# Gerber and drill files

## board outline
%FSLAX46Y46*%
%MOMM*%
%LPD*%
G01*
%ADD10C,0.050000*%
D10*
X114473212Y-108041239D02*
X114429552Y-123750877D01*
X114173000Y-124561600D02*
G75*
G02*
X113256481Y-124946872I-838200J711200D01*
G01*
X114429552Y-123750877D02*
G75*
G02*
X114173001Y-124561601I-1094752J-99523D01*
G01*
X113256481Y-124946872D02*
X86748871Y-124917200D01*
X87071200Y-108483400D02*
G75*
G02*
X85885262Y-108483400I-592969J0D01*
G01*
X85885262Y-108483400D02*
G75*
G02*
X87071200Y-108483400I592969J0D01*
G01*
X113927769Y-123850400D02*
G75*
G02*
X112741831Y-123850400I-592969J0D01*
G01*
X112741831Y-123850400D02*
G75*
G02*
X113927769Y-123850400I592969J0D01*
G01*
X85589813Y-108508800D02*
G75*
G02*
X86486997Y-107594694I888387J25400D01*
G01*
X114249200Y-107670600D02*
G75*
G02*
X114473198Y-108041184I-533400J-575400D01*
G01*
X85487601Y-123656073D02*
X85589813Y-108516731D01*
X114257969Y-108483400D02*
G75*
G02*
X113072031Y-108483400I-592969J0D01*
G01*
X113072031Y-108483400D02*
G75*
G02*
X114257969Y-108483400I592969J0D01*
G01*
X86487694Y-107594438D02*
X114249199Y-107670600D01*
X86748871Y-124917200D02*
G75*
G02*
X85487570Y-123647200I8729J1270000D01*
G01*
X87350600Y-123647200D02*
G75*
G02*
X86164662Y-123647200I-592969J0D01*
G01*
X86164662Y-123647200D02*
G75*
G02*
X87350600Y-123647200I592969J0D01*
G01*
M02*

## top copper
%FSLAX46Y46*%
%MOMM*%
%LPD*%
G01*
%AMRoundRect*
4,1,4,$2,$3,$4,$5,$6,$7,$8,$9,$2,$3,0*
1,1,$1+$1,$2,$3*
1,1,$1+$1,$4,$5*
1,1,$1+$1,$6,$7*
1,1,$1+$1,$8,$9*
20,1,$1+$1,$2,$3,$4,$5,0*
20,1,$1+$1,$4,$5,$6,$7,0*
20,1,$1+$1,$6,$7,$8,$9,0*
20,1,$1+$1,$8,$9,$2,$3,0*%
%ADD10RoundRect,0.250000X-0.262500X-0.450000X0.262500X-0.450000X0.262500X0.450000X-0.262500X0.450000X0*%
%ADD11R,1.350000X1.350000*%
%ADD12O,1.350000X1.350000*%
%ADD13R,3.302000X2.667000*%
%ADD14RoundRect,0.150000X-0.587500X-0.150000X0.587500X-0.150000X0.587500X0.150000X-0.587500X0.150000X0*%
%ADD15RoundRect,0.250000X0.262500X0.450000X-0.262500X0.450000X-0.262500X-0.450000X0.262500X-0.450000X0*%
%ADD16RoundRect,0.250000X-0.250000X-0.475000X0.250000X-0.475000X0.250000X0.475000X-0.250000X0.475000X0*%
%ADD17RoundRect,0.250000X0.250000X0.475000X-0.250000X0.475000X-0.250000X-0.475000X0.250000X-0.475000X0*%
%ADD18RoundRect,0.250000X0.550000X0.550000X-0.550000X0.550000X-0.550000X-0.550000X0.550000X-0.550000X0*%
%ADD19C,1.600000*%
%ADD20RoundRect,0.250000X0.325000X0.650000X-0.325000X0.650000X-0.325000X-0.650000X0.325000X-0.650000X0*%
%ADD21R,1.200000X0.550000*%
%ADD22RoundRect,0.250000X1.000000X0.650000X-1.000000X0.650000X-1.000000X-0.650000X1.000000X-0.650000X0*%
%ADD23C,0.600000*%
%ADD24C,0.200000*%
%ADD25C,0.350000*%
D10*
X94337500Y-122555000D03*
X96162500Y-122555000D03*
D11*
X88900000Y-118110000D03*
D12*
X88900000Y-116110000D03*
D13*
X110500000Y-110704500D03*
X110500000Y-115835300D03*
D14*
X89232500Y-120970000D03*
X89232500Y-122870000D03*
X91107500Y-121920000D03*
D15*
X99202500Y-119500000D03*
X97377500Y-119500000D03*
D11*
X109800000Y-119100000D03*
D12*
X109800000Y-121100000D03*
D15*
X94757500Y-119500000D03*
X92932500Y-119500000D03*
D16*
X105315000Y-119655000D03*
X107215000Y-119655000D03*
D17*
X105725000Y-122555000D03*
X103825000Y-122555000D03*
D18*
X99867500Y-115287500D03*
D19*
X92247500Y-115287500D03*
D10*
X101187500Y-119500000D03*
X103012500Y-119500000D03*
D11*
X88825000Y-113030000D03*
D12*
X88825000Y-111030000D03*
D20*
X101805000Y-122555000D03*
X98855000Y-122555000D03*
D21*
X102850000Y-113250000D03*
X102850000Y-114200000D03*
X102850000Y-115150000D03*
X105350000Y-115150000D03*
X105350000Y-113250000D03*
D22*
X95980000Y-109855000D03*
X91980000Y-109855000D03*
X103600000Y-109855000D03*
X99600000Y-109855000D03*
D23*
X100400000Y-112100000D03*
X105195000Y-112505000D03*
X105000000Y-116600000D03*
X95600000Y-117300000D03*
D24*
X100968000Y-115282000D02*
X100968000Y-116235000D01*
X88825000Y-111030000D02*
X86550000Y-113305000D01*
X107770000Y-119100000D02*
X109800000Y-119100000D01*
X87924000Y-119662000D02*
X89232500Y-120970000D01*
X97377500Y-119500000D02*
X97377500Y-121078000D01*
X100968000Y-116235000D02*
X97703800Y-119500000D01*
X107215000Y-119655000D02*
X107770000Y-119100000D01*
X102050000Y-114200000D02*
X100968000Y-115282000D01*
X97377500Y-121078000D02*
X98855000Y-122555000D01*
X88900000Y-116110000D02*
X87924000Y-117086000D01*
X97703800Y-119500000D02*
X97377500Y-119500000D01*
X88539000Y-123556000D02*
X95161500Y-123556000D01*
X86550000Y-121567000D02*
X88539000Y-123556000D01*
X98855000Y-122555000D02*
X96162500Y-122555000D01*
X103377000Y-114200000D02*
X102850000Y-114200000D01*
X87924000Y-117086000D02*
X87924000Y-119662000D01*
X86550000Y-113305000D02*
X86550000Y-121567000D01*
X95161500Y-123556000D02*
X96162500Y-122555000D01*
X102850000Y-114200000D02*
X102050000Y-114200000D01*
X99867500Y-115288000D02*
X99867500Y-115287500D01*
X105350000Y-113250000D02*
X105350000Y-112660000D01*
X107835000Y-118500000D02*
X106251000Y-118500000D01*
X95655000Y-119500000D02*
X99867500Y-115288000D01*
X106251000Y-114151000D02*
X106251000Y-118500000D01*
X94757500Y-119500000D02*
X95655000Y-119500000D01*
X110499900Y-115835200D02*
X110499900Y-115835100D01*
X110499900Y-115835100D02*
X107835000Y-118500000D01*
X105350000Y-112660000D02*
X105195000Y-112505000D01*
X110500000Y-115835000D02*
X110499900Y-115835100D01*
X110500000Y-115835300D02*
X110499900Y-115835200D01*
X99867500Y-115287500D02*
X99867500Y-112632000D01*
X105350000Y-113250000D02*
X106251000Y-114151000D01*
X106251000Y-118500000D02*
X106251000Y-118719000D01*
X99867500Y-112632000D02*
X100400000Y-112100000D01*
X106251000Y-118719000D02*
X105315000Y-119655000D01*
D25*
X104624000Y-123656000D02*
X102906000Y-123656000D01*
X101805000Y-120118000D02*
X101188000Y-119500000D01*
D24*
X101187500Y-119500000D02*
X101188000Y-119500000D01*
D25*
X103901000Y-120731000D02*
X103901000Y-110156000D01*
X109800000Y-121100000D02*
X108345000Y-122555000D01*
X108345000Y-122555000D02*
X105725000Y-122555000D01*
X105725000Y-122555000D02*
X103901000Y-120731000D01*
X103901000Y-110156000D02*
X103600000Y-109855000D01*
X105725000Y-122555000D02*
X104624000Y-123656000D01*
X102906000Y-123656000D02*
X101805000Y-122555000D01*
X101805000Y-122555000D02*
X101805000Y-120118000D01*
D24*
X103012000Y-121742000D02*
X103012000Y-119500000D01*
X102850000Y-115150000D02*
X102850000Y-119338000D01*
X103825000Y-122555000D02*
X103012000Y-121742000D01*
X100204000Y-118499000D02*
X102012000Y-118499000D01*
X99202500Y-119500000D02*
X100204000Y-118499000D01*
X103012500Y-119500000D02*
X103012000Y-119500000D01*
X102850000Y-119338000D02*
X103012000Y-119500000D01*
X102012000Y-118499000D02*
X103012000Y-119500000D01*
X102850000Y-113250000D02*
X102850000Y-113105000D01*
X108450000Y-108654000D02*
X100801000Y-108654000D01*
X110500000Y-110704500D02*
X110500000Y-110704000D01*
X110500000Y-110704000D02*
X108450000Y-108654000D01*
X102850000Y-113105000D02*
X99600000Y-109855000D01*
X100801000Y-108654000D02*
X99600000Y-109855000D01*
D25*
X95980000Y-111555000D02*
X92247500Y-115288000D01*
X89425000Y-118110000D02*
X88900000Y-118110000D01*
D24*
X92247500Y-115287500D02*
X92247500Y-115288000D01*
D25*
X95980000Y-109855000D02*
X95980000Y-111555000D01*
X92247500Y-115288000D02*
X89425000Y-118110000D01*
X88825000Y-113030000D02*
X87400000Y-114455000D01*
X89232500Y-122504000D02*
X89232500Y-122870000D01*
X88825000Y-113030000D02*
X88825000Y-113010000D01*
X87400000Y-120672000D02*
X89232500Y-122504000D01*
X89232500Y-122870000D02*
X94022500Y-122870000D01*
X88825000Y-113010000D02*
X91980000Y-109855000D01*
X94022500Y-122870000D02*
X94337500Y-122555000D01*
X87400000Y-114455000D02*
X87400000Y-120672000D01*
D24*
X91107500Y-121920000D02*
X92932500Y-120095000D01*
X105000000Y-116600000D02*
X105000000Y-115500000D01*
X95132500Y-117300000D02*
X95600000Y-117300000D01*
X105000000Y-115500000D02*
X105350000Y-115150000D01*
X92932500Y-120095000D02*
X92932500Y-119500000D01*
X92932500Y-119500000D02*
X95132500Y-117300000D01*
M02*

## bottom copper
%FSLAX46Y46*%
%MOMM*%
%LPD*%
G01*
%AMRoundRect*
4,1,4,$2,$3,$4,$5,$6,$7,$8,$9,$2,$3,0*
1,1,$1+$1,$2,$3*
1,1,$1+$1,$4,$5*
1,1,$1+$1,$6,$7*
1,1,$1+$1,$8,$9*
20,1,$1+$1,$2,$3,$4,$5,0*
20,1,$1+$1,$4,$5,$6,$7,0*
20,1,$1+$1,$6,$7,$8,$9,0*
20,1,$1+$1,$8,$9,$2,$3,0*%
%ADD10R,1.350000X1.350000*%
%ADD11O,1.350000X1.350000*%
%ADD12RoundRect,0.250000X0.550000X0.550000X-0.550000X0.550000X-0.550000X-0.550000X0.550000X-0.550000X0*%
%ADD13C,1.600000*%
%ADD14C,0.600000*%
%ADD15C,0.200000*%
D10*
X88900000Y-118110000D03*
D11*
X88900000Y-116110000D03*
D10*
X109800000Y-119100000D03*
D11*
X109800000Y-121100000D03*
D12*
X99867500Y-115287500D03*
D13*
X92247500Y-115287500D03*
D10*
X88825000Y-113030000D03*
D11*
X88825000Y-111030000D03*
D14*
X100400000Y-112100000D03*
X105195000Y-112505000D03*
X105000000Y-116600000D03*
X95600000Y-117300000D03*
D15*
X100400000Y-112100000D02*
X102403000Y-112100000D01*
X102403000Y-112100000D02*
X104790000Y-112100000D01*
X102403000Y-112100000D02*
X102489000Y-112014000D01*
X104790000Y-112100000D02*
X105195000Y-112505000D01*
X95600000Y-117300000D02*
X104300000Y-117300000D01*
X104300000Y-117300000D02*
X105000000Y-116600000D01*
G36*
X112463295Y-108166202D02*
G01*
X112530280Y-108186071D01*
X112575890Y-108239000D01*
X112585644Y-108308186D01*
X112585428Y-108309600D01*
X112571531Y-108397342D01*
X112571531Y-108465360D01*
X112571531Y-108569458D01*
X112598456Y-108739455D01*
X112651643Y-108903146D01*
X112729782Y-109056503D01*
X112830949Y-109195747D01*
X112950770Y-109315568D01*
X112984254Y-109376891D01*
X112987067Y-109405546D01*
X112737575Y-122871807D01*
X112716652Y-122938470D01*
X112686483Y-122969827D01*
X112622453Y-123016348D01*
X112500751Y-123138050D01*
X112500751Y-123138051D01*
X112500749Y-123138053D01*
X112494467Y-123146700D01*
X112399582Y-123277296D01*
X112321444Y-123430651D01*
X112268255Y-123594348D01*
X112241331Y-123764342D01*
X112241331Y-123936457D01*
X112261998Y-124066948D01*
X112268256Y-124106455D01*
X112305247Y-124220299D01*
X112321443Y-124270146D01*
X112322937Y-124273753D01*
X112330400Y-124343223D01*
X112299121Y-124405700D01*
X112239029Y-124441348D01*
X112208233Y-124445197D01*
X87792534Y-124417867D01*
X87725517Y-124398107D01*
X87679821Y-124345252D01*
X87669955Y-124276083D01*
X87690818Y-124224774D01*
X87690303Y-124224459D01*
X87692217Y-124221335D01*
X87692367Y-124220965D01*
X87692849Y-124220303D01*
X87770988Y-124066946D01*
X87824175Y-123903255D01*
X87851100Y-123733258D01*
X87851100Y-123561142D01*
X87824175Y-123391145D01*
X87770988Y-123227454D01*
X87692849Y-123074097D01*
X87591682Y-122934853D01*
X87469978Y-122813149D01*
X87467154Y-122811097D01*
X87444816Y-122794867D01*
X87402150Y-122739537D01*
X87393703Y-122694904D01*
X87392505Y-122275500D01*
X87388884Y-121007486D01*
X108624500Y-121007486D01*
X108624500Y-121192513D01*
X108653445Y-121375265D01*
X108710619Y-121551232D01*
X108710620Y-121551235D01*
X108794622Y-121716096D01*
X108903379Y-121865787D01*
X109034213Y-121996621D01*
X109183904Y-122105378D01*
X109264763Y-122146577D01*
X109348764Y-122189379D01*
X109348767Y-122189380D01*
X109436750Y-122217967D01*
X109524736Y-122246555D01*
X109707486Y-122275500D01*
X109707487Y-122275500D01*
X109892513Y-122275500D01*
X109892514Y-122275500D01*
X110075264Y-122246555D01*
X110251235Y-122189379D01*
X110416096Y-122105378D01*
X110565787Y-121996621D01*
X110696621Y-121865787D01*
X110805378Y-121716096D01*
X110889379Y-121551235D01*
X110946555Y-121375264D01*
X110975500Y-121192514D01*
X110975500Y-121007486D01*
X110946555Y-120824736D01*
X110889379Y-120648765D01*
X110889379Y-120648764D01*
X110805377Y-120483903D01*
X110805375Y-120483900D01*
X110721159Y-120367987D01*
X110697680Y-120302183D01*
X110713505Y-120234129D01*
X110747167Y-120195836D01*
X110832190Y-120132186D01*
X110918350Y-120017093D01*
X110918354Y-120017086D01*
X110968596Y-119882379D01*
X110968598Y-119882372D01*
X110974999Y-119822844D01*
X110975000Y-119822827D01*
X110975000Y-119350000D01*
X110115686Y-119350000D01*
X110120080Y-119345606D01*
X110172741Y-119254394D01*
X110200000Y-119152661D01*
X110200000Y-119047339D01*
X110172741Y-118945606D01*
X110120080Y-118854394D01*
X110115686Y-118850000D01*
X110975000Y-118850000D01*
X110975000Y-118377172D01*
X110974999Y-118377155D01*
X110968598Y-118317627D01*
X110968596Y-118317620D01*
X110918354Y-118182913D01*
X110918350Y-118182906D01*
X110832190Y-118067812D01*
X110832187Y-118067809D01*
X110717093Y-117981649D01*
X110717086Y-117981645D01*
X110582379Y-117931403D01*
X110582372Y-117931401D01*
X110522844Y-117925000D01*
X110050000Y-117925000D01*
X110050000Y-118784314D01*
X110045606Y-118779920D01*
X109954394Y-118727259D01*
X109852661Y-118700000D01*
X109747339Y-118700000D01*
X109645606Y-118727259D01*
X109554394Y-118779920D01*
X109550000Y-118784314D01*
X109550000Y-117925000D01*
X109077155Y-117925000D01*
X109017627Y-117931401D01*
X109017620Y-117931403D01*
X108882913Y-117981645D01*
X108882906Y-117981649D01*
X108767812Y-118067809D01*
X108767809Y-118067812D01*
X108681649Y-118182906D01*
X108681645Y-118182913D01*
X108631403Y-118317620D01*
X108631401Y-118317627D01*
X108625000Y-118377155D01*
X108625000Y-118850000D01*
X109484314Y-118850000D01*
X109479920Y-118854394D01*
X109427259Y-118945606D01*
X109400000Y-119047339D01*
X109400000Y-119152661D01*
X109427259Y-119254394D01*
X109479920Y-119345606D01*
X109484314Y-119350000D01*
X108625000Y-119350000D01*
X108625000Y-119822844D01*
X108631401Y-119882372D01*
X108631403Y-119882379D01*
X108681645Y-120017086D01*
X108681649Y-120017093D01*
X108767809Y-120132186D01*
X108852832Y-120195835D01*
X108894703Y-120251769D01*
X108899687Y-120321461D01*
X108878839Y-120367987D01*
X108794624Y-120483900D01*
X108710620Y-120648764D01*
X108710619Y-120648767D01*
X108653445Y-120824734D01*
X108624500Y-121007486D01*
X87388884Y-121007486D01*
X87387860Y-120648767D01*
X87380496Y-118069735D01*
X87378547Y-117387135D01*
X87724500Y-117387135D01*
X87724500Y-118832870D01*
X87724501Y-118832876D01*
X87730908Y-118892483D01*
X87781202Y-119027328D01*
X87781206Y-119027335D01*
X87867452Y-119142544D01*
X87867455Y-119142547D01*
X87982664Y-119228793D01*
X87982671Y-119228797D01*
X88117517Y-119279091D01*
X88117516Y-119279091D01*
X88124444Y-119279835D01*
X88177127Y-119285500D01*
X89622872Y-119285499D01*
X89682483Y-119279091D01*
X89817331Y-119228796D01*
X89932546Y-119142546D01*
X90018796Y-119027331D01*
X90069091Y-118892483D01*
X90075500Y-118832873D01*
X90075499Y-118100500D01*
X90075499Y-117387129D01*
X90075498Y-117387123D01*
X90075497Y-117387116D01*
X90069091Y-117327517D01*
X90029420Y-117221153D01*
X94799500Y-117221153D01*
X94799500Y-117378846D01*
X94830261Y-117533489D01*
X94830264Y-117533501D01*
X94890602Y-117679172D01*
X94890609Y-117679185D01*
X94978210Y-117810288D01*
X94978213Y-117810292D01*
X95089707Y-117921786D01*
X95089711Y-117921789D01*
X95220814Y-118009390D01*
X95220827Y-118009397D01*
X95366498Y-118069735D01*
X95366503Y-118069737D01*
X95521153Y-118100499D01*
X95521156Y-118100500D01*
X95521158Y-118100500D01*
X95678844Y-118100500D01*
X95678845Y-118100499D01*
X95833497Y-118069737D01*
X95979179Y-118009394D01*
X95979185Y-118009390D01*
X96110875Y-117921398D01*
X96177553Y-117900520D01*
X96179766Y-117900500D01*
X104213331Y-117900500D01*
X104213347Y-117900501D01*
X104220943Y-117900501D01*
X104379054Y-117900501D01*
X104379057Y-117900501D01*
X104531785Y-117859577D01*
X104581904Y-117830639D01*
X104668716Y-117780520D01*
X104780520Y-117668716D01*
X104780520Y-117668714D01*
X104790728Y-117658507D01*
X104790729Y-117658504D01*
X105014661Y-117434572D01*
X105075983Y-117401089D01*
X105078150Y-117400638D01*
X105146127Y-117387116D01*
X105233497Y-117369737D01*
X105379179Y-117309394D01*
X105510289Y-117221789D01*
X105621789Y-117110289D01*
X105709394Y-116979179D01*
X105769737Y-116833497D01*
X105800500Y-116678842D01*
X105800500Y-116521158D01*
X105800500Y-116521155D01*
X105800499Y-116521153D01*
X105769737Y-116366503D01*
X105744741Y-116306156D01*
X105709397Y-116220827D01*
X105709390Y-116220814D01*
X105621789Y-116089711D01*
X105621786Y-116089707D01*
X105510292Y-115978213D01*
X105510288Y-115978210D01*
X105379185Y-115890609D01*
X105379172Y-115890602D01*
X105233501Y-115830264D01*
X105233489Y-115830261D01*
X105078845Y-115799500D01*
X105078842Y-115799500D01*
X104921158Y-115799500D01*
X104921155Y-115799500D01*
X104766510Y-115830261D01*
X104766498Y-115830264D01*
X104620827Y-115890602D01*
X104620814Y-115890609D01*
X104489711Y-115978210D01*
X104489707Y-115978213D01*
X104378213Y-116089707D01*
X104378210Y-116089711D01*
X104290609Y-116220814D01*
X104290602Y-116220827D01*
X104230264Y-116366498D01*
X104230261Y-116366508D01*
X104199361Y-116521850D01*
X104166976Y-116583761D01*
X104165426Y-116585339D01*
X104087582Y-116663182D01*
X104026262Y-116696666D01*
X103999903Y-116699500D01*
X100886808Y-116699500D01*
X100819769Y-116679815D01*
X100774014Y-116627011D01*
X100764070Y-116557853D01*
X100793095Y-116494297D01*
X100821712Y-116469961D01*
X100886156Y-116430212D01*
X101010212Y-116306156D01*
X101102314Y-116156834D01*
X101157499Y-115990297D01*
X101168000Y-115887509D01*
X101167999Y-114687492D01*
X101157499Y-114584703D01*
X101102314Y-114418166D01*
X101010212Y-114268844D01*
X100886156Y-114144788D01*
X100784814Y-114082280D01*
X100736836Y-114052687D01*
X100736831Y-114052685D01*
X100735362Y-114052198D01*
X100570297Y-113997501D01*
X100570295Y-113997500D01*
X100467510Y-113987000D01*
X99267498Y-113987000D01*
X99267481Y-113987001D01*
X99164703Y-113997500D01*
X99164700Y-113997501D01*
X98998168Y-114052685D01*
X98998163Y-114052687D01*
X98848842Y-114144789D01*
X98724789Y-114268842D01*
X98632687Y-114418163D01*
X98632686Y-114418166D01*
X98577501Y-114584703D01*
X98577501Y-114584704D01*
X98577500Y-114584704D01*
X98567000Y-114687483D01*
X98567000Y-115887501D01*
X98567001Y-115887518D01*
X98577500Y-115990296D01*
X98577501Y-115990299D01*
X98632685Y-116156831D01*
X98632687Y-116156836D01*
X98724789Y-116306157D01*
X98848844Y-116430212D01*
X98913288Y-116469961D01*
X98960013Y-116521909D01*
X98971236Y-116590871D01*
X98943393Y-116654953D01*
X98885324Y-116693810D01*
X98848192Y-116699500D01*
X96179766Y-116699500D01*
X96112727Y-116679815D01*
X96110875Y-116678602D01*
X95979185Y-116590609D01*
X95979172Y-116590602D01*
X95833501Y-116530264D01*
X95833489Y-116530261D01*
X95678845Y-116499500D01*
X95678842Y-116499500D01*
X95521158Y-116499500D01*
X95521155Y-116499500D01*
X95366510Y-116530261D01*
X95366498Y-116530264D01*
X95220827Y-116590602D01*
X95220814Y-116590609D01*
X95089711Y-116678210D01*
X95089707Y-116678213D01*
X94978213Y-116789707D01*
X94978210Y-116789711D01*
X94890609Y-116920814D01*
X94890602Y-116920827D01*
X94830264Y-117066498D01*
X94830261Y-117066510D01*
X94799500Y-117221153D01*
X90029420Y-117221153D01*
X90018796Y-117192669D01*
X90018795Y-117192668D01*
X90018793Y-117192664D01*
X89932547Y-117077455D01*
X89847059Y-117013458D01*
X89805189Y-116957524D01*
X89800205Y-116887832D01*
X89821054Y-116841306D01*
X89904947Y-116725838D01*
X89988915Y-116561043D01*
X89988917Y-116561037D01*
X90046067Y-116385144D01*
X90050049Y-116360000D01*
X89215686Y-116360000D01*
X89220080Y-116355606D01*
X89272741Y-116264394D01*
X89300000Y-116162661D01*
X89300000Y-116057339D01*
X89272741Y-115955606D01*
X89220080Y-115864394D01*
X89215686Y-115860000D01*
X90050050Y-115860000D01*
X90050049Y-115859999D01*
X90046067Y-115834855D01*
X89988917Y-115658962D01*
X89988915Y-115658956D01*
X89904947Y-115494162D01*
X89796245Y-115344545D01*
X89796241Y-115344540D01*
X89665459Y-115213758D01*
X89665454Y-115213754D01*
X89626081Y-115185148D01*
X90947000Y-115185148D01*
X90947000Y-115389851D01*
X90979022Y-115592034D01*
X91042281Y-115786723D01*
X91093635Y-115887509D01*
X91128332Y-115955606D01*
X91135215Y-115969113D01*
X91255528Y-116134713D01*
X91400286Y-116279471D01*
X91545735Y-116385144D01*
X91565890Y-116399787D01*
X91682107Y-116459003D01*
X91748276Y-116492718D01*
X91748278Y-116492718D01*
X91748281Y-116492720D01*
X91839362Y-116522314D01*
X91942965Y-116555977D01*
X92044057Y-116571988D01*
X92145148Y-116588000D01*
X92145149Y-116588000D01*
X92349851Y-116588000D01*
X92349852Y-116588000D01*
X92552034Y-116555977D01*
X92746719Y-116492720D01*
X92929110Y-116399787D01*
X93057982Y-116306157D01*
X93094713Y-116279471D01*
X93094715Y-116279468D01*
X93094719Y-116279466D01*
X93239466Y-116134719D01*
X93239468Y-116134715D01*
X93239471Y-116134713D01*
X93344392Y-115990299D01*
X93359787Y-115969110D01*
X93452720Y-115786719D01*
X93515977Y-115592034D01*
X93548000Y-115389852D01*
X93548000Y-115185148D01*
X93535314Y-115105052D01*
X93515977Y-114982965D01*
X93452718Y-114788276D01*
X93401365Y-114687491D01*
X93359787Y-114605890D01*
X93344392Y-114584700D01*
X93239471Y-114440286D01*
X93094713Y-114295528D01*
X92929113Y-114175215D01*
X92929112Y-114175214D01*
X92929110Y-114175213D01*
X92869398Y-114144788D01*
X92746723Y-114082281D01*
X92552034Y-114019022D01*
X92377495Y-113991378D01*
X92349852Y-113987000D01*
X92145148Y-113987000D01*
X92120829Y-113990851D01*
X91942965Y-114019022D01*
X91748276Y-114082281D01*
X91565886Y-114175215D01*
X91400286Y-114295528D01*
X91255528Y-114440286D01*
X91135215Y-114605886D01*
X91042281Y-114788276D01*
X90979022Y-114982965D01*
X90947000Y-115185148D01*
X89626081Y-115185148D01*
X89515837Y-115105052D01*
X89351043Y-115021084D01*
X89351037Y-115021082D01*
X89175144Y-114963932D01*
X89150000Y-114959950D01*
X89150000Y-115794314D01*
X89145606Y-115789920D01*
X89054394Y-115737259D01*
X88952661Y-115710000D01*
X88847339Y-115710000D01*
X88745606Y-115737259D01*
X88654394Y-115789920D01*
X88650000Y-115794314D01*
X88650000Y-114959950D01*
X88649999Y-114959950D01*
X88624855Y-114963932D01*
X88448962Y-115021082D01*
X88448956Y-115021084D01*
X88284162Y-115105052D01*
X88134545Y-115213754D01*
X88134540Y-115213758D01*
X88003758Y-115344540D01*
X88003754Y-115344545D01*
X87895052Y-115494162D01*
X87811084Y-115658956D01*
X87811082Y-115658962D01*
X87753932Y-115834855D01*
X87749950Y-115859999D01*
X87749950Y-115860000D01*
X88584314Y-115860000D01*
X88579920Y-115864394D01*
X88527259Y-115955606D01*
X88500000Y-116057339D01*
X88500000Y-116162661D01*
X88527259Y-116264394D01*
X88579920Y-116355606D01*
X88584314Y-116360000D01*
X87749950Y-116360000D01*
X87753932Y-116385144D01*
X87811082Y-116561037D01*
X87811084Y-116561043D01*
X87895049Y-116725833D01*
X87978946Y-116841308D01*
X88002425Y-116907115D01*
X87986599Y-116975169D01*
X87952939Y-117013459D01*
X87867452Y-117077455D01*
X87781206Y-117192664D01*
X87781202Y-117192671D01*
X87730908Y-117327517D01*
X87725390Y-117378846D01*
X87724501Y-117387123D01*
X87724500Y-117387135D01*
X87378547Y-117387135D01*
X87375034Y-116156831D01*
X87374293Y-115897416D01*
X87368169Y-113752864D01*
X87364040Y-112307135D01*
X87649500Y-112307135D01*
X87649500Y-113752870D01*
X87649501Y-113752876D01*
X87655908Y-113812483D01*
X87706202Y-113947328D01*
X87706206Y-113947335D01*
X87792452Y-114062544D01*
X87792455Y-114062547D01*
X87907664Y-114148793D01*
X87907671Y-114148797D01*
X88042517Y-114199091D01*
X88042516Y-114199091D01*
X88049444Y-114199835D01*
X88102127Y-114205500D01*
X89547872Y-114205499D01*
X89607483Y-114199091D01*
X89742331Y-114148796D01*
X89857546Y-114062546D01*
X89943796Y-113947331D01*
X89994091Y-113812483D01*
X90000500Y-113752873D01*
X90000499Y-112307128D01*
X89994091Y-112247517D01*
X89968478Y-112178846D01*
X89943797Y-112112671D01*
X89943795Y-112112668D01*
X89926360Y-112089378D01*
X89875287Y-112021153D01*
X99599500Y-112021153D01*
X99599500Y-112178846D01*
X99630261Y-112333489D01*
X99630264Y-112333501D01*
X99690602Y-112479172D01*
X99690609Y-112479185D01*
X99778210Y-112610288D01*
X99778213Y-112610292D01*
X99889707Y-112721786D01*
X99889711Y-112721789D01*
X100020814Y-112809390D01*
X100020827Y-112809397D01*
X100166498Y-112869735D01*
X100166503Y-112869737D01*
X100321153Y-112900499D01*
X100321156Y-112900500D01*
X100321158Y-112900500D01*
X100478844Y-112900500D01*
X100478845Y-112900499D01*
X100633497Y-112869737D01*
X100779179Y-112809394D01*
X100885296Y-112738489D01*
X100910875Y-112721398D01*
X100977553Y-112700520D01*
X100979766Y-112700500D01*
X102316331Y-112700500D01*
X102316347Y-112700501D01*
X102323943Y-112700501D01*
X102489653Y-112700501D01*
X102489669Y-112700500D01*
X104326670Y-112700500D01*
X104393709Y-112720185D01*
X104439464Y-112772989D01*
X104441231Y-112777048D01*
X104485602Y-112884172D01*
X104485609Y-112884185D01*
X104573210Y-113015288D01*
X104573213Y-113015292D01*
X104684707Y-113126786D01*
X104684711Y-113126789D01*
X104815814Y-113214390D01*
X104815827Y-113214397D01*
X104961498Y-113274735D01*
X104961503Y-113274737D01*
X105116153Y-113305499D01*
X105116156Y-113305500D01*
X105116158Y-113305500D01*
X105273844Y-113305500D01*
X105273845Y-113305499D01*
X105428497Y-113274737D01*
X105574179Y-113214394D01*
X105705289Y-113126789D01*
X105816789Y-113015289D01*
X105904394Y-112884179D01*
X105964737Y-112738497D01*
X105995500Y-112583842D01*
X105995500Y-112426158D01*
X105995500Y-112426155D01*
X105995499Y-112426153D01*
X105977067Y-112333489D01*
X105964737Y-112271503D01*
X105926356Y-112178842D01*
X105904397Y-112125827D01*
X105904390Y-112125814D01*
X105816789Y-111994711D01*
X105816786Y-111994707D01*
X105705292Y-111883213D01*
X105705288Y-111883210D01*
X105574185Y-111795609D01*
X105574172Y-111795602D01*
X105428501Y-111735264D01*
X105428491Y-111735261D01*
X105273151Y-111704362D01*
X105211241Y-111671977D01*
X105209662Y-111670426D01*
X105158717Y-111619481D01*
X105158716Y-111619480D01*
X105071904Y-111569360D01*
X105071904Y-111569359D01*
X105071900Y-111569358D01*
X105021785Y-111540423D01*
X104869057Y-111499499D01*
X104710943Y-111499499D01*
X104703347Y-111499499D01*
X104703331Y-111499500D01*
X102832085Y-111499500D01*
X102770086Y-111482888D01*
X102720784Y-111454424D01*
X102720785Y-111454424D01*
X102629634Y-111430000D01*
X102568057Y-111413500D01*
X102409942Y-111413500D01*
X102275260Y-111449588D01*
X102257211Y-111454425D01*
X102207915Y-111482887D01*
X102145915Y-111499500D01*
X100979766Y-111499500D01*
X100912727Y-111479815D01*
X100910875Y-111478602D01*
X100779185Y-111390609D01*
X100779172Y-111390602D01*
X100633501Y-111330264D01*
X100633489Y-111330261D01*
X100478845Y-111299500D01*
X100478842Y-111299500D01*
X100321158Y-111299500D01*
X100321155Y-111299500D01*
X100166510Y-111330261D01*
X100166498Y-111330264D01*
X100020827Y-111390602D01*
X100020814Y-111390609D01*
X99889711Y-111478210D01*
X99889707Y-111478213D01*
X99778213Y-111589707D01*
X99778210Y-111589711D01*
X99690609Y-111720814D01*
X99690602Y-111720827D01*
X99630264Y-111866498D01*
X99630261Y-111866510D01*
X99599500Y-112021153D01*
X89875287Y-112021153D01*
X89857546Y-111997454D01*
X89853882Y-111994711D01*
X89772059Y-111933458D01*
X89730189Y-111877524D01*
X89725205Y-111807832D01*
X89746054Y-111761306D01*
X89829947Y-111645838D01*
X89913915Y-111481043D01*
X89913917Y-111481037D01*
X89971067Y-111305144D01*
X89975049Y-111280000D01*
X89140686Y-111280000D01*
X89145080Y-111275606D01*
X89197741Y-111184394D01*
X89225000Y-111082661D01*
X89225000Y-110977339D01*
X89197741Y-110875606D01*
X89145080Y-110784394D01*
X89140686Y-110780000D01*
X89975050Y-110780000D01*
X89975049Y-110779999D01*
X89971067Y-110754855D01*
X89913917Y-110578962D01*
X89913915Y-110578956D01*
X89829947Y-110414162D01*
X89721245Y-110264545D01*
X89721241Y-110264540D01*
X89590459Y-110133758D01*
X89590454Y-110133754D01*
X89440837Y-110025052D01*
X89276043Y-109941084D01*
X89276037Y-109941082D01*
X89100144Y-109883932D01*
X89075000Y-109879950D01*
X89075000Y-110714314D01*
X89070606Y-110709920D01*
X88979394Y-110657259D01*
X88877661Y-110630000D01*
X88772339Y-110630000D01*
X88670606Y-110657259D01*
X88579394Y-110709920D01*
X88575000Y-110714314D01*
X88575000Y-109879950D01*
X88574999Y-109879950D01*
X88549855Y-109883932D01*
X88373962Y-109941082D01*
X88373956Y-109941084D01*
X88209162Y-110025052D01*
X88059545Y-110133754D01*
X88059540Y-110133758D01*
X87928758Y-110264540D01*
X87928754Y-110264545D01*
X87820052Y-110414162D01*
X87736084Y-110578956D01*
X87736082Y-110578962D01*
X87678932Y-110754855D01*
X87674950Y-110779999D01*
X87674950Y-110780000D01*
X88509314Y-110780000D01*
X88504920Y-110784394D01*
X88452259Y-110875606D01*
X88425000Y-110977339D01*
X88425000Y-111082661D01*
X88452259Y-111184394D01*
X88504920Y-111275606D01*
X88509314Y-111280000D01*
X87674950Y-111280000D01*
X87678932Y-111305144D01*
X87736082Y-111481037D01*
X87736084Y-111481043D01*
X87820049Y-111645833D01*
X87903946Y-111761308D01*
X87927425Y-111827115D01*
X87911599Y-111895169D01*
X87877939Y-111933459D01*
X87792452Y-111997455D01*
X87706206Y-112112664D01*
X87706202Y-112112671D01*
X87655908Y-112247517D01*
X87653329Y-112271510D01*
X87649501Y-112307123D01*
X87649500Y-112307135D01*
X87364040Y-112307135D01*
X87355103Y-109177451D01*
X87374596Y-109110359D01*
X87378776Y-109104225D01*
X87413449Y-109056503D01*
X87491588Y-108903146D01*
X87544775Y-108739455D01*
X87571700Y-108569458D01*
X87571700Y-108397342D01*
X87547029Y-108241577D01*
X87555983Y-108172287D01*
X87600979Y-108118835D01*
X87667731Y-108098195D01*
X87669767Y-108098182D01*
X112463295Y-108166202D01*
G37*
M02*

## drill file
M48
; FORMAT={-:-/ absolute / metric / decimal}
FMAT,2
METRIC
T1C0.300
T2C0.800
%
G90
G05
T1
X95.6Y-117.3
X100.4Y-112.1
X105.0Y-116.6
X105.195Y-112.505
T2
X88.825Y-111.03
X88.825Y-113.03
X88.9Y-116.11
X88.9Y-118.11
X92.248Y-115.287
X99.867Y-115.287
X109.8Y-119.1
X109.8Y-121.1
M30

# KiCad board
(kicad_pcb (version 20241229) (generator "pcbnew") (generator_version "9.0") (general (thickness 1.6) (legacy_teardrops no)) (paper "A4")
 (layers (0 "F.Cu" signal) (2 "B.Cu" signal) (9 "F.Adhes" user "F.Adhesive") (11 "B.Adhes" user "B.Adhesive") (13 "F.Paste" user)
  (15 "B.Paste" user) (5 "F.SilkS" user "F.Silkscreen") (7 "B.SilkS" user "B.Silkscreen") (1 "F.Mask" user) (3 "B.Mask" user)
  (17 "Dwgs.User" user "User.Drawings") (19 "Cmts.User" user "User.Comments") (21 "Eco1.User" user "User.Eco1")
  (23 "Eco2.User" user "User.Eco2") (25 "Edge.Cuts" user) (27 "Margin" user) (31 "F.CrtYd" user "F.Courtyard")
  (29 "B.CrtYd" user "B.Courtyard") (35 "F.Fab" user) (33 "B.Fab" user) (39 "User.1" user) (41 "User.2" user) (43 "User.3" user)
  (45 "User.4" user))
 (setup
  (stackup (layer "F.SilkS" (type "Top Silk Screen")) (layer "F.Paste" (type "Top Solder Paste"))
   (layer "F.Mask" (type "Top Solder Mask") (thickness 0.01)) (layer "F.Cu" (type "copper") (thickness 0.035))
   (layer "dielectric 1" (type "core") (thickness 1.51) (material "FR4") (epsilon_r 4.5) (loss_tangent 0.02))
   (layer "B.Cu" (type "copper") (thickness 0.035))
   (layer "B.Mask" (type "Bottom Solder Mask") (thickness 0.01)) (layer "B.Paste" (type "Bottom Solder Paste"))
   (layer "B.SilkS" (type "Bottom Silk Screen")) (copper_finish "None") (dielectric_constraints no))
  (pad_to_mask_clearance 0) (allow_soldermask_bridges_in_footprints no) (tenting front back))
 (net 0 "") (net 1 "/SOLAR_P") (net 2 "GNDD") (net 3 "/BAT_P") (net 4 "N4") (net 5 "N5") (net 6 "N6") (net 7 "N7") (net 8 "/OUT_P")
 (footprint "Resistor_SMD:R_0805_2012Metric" (layer "F.Cu") (at 95.25 122.555)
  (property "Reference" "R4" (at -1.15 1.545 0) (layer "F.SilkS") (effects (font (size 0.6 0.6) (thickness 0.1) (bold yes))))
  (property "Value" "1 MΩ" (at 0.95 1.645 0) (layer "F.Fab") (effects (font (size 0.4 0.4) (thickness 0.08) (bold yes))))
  (pad "1" smd roundrect (at -0.9125 0) (size 1.025 1.4) (layers "F.Cu" "F.Mask" "F.Paste") (roundrect_rratio 0.243902) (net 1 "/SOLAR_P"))
  (pad "2" smd roundrect (at 0.9125 0) (size 1.025 1.4) (layers "F.Cu" "F.Mask" "F.Paste") (roundrect_rratio 0.243902) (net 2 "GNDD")))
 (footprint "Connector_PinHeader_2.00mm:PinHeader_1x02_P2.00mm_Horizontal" (layer "F.Cu") (at 88.9 118.11 180)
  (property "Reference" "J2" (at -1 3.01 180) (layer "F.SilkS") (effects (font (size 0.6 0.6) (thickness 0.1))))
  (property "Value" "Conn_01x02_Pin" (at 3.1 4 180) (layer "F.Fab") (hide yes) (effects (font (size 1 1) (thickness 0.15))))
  (pad "1" thru_hole rect (at 0 0 180) (size 1.35 1.35) (drill 0.8) (layers "*.Cu" "*.Mask") (remove_unused_layers no) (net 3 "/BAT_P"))
  (pad "2" thru_hole oval (at 0 2 180) (size 1.35 1.35) (drill 0.8) (layers "*.Cu" "*.Mask") (remove_unused_layers no) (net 2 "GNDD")))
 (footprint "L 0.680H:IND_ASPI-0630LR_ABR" (layer "F.Cu") (at 110.5 113.2699 -90)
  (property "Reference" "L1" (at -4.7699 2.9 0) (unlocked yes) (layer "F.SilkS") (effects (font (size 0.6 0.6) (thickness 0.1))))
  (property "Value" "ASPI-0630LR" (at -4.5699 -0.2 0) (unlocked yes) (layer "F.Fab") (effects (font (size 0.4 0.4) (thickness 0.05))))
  (pad "1" smd rect (at -2.5654 0) (size 3.302 2.667) (layers "F.Cu" "F.Mask" "F.Paste") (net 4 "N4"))
  (pad "2" smd rect (at 2.5654 0) (size 3.302 2.667) (layers "F.Cu" "F.Mask" "F.Paste") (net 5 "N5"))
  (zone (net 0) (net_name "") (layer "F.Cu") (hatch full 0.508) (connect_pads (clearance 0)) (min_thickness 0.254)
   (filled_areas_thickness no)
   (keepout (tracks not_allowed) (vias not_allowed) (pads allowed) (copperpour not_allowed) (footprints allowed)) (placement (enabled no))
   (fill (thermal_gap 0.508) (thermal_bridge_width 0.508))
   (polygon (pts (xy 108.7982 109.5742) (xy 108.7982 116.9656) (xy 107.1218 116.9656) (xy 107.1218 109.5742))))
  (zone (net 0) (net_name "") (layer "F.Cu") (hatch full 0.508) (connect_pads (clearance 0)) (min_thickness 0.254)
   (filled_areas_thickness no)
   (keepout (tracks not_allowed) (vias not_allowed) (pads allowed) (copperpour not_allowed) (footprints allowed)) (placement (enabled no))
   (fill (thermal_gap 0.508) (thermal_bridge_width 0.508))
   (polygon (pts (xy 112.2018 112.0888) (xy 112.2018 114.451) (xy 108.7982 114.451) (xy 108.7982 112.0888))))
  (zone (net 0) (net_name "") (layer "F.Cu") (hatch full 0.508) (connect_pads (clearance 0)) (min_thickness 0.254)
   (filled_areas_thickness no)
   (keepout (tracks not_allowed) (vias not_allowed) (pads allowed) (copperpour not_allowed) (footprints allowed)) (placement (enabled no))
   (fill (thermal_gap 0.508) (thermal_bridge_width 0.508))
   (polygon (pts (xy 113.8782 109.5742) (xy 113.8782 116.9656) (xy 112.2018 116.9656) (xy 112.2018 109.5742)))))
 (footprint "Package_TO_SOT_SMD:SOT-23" (layer "F.Cu") (at 90.17 121.92)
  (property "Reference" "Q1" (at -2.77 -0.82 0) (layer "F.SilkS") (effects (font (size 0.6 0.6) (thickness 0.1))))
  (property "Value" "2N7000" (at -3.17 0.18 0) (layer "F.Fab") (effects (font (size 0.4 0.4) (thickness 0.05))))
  (pad "1" smd roundrect (at -0.9375 -0.95) (size 1.475 0.6) (layers "F.Cu" "F.Mask" "F.Paste") (roundrect_rratio 0.25) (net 2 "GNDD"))
  (pad "2" smd roundrect (at -0.9375 0.95) (size 1.475 0.6) (layers "F.Cu" "F.Mask" "F.Paste") (roundrect_rratio 0.25) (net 1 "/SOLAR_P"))
  (pad "3" smd roundrect (at 0.9375 0) (size 1.475 0.6) (layers "F.Cu" "F.Mask" "F.Paste") (roundrect_rratio 0.25) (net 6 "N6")))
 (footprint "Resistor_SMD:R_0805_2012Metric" (layer "F.Cu") (at 98.29 119.5 180)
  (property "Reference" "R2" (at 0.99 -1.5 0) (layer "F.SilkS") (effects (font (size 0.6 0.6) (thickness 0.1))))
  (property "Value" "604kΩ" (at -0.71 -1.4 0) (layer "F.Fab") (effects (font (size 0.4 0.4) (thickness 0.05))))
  (pad "1" smd roundrect (at -0.9125 0 180) (size 1.025 1.4) (layers "F.Cu" "F.Mask" "F.Paste") (roundrect_rratio 0.243902) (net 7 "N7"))
  (pad "2" smd roundrect (at 0.9125 0 180) (size 1.025 1.4) (layers "F.Cu" "F.Mask" "F.Paste") (roundrect_rratio 0.243902) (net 2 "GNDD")))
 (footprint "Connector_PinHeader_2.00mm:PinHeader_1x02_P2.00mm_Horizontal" (layer "F.Cu") (at 109.8 119.1)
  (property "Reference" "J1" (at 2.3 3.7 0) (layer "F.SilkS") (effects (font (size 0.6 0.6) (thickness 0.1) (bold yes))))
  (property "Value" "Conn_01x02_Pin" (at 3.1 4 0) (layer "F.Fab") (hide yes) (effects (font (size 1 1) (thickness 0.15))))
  (pad "1" thru_hole rect (at 0 0) (size 1.35 1.35) (drill 0.8) (layers "*.Cu" "*.Mask") (remove_unused_layers no) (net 2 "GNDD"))
  (pad "2" thru_hole oval (at 0 2) (size 1.35 1.35) (drill 0.8) (layers "*.Cu" "*.Mask") (remove_unused_layers no) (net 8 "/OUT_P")))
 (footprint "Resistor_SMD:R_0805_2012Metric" (layer "F.Cu") (at 93.845 119.5 180)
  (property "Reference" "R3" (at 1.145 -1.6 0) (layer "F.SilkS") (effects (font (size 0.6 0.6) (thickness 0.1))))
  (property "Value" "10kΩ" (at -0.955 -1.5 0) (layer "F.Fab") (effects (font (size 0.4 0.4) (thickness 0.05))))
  (pad "1" smd roundrect (at -0.9125 0 180) (size 1.025 1.4) (layers "F.Cu" "F.Mask" "F.Paste") (roundrect_rratio 0.243902) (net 5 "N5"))
  (pad "2" smd roundrect (at 0.9125 0 180) (size 1.025 1.4) (layers "F.Cu" "F.Mask" "F.Paste") (roundrect_rratio 0.243902) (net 6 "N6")))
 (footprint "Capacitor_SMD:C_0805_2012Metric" (layer "F.Cu") (at 106.265 119.655)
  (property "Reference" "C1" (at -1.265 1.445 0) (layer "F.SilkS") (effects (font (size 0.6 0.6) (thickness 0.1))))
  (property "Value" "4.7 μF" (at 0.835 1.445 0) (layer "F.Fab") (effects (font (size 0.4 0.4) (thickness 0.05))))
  (pad "1" smd roundrect (at -0.95 0) (size 1 1.45) (layers "F.Cu" "F.Mask" "F.Paste") (roundrect_rratio 0.25) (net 5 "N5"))
  (pad "2" smd roundrect (at 0.95 0) (size 1 1.45) (layers "F.Cu" "F.Mask" "F.Paste") (roundrect_rratio 0.25) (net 2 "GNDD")))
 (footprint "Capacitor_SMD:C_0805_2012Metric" (layer "F.Cu") (at 104.775 122.555 180)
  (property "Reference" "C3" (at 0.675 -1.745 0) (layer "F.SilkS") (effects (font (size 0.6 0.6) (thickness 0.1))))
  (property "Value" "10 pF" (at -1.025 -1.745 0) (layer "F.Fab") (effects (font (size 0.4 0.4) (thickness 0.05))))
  (pad "1" smd roundrect (at -0.95 0 180) (size 1 1.45) (layers "F.Cu" "F.Mask" "F.Paste") (roundrect_rratio 0.25) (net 8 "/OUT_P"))
  (pad "2" smd roundrect (at 0.95 0 180) (size 1 1.45) (layers "F.Cu" "F.Mask" "F.Paste") (roundrect_rratio 0.25) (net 7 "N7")))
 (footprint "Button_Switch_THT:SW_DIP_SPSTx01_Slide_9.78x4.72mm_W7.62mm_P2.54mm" (layer "F.Cu") (at 99.8675 115.2875 180)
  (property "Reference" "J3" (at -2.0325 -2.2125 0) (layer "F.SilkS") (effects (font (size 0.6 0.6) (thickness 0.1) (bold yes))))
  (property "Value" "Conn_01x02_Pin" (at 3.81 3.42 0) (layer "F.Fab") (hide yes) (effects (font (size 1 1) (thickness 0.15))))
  (pad "1" thru_hole roundrect (at 0 0 180) (size 1.6 1.6) (drill 0.8) (layers "*.Cu" "*.Mask") (remove_unused_layers no)
   (roundrect_rratio 0.15625) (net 5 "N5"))
  (pad "2" thru_hole circle (at 7.62 0 180) (size 1.6 1.6) (drill 0.8) (layers "*.Cu" "*.Mask") (remove_unused_layers no) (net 3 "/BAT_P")))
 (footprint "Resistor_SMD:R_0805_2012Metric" (layer "F.Cu") (at 102.1 119.5)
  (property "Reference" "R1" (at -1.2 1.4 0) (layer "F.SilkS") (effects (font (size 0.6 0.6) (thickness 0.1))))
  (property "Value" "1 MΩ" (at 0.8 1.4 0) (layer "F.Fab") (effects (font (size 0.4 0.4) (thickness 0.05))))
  (pad "1" smd roundrect (at -0.9125 0) (size 1.025 1.4) (layers "F.Cu" "F.Mask" "F.Paste") (roundrect_rratio 0.243902) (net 8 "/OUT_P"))
  (pad "2" smd roundrect (at 0.9125 0) (size 1.025 1.4) (layers "F.Cu" "F.Mask" "F.Paste") (roundrect_rratio 0.243902) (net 7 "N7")))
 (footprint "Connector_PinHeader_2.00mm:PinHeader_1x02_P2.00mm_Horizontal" (layer "F.Cu") (at 88.825 113.03 180)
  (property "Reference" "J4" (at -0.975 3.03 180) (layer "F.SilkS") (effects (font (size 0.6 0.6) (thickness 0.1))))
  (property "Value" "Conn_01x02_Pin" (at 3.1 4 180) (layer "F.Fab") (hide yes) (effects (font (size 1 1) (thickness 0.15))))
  (pad "1" thru_hole rect (at 0 0 180) (size 1.35 1.35) (drill 0.8) (layers "*.Cu" "*.Mask") (remove_unused_layers no) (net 1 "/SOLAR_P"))
  (pad "2" thru_hole oval (at 0 2 180) (size 1.35 1.35) (drill 0.8) (layers "*.Cu" "*.Mask") (remove_unused_layers no) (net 2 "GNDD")))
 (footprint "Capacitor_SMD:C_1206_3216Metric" (layer "F.Cu") (at 100.33 122.555 180)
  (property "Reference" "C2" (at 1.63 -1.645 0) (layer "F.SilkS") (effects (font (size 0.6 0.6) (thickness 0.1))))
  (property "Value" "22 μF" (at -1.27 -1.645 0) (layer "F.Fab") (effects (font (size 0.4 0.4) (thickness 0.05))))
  (pad "1" smd roundrect (at -1.475 0 180) (size 1.15 1.8) (layers "F.Cu" "F.Mask" "F.Paste") (roundrect_rratio 0.217391) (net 8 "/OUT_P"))
  (pad "2" smd roundrect (at 1.475 0 180) (size 1.15 1.8) (layers "F.Cu" "F.Mask" "F.Paste") (roundrect_rratio 0.217391) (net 2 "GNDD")))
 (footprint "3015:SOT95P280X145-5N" (layer "F.Cu") (at 104.1 114.2)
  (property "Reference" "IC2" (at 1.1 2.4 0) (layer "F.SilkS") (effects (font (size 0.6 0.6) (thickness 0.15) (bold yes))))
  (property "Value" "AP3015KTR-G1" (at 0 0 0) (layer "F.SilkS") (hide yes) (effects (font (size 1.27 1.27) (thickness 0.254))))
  (pad "1" smd rect (at -1.25 -0.95 90) (size 0.55 1.2) (layers "F.Cu" "F.Mask" "F.Paste") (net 4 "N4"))
  (pad "2" smd rect (at -1.25 0 90) (size 0.55 1.2) (layers "F.Cu" "F.Mask" "F.Paste") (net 2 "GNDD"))
  (pad "3" smd rect (at -1.25 0.95 90) (size 0.55 1.2) (layers "F.Cu" "F.Mask" "F.Paste") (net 7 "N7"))
  (pad "4" smd rect (at 1.25 0.95 90) (size 0.55 1.2) (layers "F.Cu" "F.Mask" "F.Paste") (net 6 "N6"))
  (pad "5" smd rect (at 1.25 -0.95 90) (size 0.55 1.2) (layers "F.Cu" "F.Mask" "F.Paste") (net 5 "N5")))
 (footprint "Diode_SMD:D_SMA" (layer "F.Cu") (at 93.98 109.855 180)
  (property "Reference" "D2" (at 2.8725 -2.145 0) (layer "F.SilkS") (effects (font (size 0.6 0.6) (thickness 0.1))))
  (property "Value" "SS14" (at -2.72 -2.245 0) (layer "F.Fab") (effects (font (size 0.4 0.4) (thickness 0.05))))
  (pad "1" smd roundrect (at -2 0 180) (size 2.5 1.8) (layers "F.Cu" "F.Mask" "F.Paste") (roundrect_rratio 0.1388888889) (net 3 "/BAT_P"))
  (pad "2" smd roundrect (at 2 0 180) (size 2.5 1.8) (layers "F.Cu" "F.Mask" "F.Paste") (roundrect_rratio 0.1388888889) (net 1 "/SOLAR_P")))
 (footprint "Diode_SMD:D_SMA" (layer "F.Cu") (at 101.6 109.855 180)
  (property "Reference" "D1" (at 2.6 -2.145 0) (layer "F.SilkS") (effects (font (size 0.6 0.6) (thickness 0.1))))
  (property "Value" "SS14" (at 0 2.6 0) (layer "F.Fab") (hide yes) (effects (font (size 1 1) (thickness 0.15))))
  (pad "1" smd roundrect (at -2 0 180) (size 2.5 1.8) (layers "F.Cu" "F.Mask" "F.Paste") (roundrect_rratio 0.1388888889) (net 8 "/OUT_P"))
  (pad "2" smd roundrect (at 2 0 180) (size 2.5 1.8) (layers "F.Cu" "F.Mask" "F.Paste") (roundrect_rratio 0.1388888889) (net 4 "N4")))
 (gr_line (start 114.473212 108.041239) (end 114.429552 123.750877) (stroke (width 0.05) (type default)) (layer "Edge.Cuts"))
 (gr_arc (start 114.173 124.5616) (mid 113.760785 124.863771) (end 113.256481 124.946872) (stroke (width 0.05) (type default))
  (layer "Edge.Cuts"))
 (gr_arc (start 114.429552 123.750877) (mid 114.382843 124.18205) (end 114.173 124.5616) (stroke (width 0.05) (type default))
  (layer "Edge.Cuts"))
 (gr_line (start 113.256481 124.946872) (end 86.748871 124.9172) (stroke (width 0.05) (type default)) (layer "Edge.Cuts"))
 (gr_circle (center 86.478231 108.4834) (end 86.884631 108.9152) (stroke (width 0.05) (type default)) (fill no) (layer "Edge.Cuts"))
 (gr_circle (center 113.3348 123.8504) (end 113.7412 124.2822) (stroke (width 0.05) (type default)) (fill no) (layer "Edge.Cuts"))
 (gr_arc (start 85.589813 108.5088) (mid 85.843913 107.860847) (end 86.486997 107.594662) (stroke (width 0.05) (type default))
  (layer "Edge.Cuts"))
 (gr_arc (start 114.2492 107.6706) (mid 114.387277 107.84013) (end 114.473212 108.04118) (stroke (width 0.05) (type default))
  (layer "Edge.Cuts"))
 (gr_line (start 85.487601 123.656073) (end 85.589813 108.516731) (stroke (width 0.05) (type default)) (layer "Edge.Cuts"))
 (gr_circle (center 113.665 108.4834) (end 114.0714 108.9152) (stroke (width 0.05) (type default)) (fill no) (layer "Edge.Cuts"))
 (gr_line (start 86.487694 107.594438) (end 114.249199 107.6706) (stroke (width 0.05) (type default)) (layer "Edge.Cuts"))
 (gr_arc (start 86.748871 124.9172) (mid 85.856492 124.542144) (end 85.487601 123.6472) (stroke (width 0.05) (type default))
  (layer "Edge.Cuts"))
 (gr_circle (center 86.757631 123.6472) (end 87.164031 124.079) (stroke (width 0.05) (type default)) (fill no) (layer "Edge.Cuts"))
 (segment (start 100.968 115.282) (end 100.968 116.235) (width 0.2) (layer "F.Cu") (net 2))
 (segment (start 88.825 111.03) (end 86.55 113.305) (width 0.2) (layer "F.Cu") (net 2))
 (segment (start 107.77 119.1) (end 109.8 119.1) (width 0.2) (layer "F.Cu") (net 2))
 (segment (start 87.924 119.662) (end 89.2325 120.97) (width 0.2) (layer "F.Cu") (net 2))
 (segment (start 97.3775 119.5) (end 97.3775 121.078) (width 0.2) (layer "F.Cu") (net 2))
 (segment (start 100.968 116.235) (end 97.7038 119.5) (width 0.2) (layer "F.Cu") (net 2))
 (segment (start 107.215 119.655) (end 107.77 119.1) (width 0.2) (layer "F.Cu") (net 2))
 (segment (start 102.05 114.2) (end 100.968 115.282) (width 0.2) (layer "F.Cu") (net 2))
 (segment (start 97.3775 121.078) (end 98.855 122.555) (width 0.2) (layer "F.Cu") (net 2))
 (segment (start 88.9 116.11) (end 87.924 117.086) (width 0.2) (layer "F.Cu") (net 2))
 (segment (start 97.7038 119.5) (end 97.3775 119.5) (width 0.2) (layer "F.Cu") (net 2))
 (segment (start 88.539 123.556) (end 95.1615 123.556) (width 0.2) (layer "F.Cu") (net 2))
 (segment (start 86.55 121.567) (end 88.539 123.556) (width 0.2) (layer "F.Cu") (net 2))
 (segment (start 98.855 122.555) (end 96.1625 122.555) (width 0.2) (layer "F.Cu") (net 2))
 (segment (start 103.377 114.2) (end 102.85 114.2) (width 0.2) (layer "F.Cu") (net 2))
 (segment (start 87.924 117.086) (end 87.924 119.662) (width 0.2) (layer "F.Cu") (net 2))
 (segment (start 86.55 113.305) (end 86.55 121.567) (width 0.2) (layer "F.Cu") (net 2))
 (segment (start 95.1615 123.556) (end 96.1625 122.555) (width 0.2) (layer "F.Cu") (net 2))
 (segment (start 102.85 114.2) (end 102.05 114.2) (width 0.2) (layer "F.Cu") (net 2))
 (segment (start 99.8675 115.288) (end 99.8675 115.2875) (width 0.2) (layer "F.Cu") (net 5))
 (segment (start 105.35 113.25) (end 105.35 112.66) (width 0.2) (layer "F.Cu") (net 5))
 (segment (start 107.835 118.5) (end 106.251 118.5) (width 0.2) (layer "F.Cu") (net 5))
 (segment (start 95.655 119.5) (end 99.8675 115.288) (width 0.2) (layer "F.Cu") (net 5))
 (segment (start 106.251 114.151) (end 106.251 118.5) (width 0.2) (layer "F.Cu") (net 5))
 (segment (start 94.7575 119.5) (end 95.655 119.5) (width 0.2) (layer "F.Cu") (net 5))
 (segment (start 110.4999 115.8352) (end 110.4999 115.8351) (width 0.2) (layer "F.Cu") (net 5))
 (segment (start 110.4999 115.8351) (end 107.835 118.5) (width 0.2) (layer "F.Cu") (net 5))
 (segment (start 105.35 112.66) (end 105.195 112.505) (width 0.2) (layer "F.Cu") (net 5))
 (segment (start 110.5 115.835) (end 110.4999 115.8351) (width 0.2) (layer "F.Cu") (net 5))
 (segment (start 110.5 115.8353) (end 110.4999 115.8352) (width 0.2) (layer "F.Cu") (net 5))
 (segment (start 99.8675 115.2875) (end 99.8675 112.632) (width 0.2) (layer "F.Cu") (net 5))
 (segment (start 105.35 113.25) (end 106.251 114.151) (width 0.2) (layer "F.Cu") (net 5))
 (segment (start 106.251 118.5) (end 106.251 118.719) (width 0.2) (layer "F.Cu") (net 5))
 (segment (start 99.8675 112.632) (end 100.4 112.1) (width 0.2) (layer "F.Cu") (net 5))
 (segment (start 106.251 118.719) (end 105.315 119.655) (width 0.2) (layer "F.Cu") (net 5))
 (via (at 100.4 112.1) (size 0.6) (drill 0.3) (layers "F.Cu" "B.Cu") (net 5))
 (via (at 105.195 112.505) (size 0.6) (drill 0.3) (layers "F.Cu" "B.Cu") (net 5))
 (segment (start 100.4 112.1) (end 102.403 112.1) (width 0.2) (layer "B.Cu") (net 5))
 (segment (start 102.403 112.1) (end 104.79 112.1) (width 0.2) (layer "B.Cu") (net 5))
 (segment (start 102.403 112.1) (end 102.489 112.014) (width 0.2) (layer "B.Cu") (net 5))
 (segment (start 104.79 112.1) (end 105.195 112.505) (width 0.2) (layer "B.Cu") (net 5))
 (segment (start 104.624 123.656) (end 102.906 123.656) (width 0.35) (layer "F.Cu") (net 8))
 (segment (start 101.805 120.118) (end 101.188 119.5) (width 0.35) (layer "F.Cu") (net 8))
 (segment (start 101.1875 119.5) (end 101.188 119.5) (width 0.2) (layer "F.Cu") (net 8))
 (segment (start 103.901 120.731) (end 103.901 110.156) (width 0.35) (layer "F.Cu") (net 8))
 (segment (start 109.8 121.1) (end 108.345 122.555) (width 0.35) (layer "F.Cu") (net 8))
 (segment (start 108.345 122.555) (end 105.725 122.555) (width 0.35) (layer "F.Cu") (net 8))
 (segment (start 105.725 122.555) (end 103.901 120.731) (width 0.35) (layer "F.Cu") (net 8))
 (segment (start 103.901 110.156) (end 103.6 109.855) (width 0.35) (layer "F.Cu") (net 8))
 (segment (start 105.725 122.555) (end 104.624 123.656) (width 0.35) (layer "F.Cu") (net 8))
 (segment (start 102.906 123.656) (end 101.805 122.555) (width 0.35) (layer "F.Cu") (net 8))
 (segment (start 101.805 122.555) (end 101.805 120.118) (width 0.35) (layer "F.Cu") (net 8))
 (segment (start 103.012 121.742) (end 103.012 119.5) (width 0.2) (layer "F.Cu") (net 7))
 (segment (start 102.85 115.15) (end 102.85 119.338) (width 0.2) (layer "F.Cu") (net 7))
 (segment (start 103.825 122.555) (end 103.012 121.742) (width 0.2) (layer "F.Cu") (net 7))
 (segment (start 100.204 118.499) (end 102.012 118.499) (width 0.2) (layer "F.Cu") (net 7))
 (segment (start 99.2025 119.5) (end 100.204 118.499) (width 0.2) (layer "F.Cu") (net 7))
 (segment (start 103.0125 119.5) (end 103.012 119.5) (width 0.2) (layer "F.Cu") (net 7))
 (segment (start 102.85 119.338) (end 103.012 119.5) (width 0.2) (layer "F.Cu") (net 7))
 (segment (start 102.012 118.499) (end 103.012 119.5) (width 0.2) (layer "F.Cu") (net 7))
 (segment (start 102.85 113.25) (end 102.85 113.105) (width 0.2) (layer "F.Cu") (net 4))
 (segment (start 108.45 108.654) (end 100.801 108.654) (width 0.2) (layer "F.Cu") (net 4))
 (segment (start 110.5 110.7045) (end 110.5 110.704) (width 0.2) (layer "F.Cu") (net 4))
 (segment (start 110.5 110.704) (end 108.45 108.654) (width 0.2) (layer "F.Cu") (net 4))
 (segment (start 102.85 113.105) (end 99.6 109.855) (width 0.2) (layer "F.Cu") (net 4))
 (segment (start 100.801 108.654) (end 99.6 109.855) (width 0.2) (layer "F.Cu") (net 4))
 (segment (start 95.98 111.555) (end 92.2475 115.288) (width 0.35) (layer "F.Cu") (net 3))
 (segment (start 89.425 118.11) (end 88.9 118.11) (width 0.35) (layer "F.Cu") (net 3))
 (segment (start 92.2475 115.2875) (end 92.2475 115.288) (width 0.2) (layer "F.Cu") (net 3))
 (segment (start 95.98 109.855) (end 95.98 111.555) (width 0.35) (layer "F.Cu") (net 3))
 (segment (start 92.2475 115.288) (end 89.425 118.11) (width 0.35) (layer "F.Cu") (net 3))
 (segment (start 88.825 113.03) (end 87.4 114.455) (width 0.35) (layer "F.Cu") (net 1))
 (segment (start 89.2325 122.504) (end 89.2325 122.87) (width 0.35) (layer "F.Cu") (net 1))
 (segment (start 88.825 113.03) (end 88.825 113.01) (width 0.35) (layer "F.Cu") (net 1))
 (segment (start 87.4 120.672) (end 89.2325 122.504) (width 0.35) (layer "F.Cu") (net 1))
 (segment (start 89.2325 122.87) (end 94.0225 122.87) (width 0.35) (layer "F.Cu") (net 1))
 (segment (start 88.825 113.01) (end 91.98 109.855) (width 0.35) (layer "F.Cu") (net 1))
 (segment (start 94.0225 122.87) (end 94.3375 122.555) (width 0.35) (layer "F.Cu") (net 1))
 (segment (start 87.4 114.455) (end 87.4 120.672) (width 0.35) (layer "F.Cu") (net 1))
 (segment (start 91.1075 121.92) (end 92.9325 120.095) (width 0.2) (layer "F.Cu") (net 6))
 (segment (start 105 116.6) (end 105 115.5) (width 0.2) (layer "F.Cu") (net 6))
 (segment (start 95.1325 117.3) (end 95.6 117.3) (width 0.2) (layer "F.Cu") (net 6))
 (segment (start 105 115.5) (end 105.35 115.15) (width 0.2) (layer "F.Cu") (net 6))
 (segment (start 92.9325 120.095) (end 92.9325 119.5) (width 0.2) (layer "F.Cu") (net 6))
 (segment (start 92.9325 119.5) (end 95.1325 117.3) (width 0.2) (layer "F.Cu") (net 6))
 (via (at 105 116.6) (size 0.6) (drill 0.3) (layers "F.Cu" "B.Cu") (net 6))
 (via (at 95.6 117.3) (size 0.6) (drill 0.3) (layers "F.Cu" "B.Cu") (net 6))
 (segment (start 95.6 117.3) (end 104.3 117.3) (width 0.2) (layer "B.Cu") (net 6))
 (segment (start 104.3 117.3) (end 105 116.6) (width 0.2) (layer "B.Cu") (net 6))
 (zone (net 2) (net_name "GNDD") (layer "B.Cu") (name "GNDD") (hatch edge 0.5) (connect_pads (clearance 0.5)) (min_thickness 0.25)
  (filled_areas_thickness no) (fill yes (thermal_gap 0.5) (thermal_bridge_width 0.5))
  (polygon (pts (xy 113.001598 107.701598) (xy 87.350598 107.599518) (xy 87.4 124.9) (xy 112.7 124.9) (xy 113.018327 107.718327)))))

